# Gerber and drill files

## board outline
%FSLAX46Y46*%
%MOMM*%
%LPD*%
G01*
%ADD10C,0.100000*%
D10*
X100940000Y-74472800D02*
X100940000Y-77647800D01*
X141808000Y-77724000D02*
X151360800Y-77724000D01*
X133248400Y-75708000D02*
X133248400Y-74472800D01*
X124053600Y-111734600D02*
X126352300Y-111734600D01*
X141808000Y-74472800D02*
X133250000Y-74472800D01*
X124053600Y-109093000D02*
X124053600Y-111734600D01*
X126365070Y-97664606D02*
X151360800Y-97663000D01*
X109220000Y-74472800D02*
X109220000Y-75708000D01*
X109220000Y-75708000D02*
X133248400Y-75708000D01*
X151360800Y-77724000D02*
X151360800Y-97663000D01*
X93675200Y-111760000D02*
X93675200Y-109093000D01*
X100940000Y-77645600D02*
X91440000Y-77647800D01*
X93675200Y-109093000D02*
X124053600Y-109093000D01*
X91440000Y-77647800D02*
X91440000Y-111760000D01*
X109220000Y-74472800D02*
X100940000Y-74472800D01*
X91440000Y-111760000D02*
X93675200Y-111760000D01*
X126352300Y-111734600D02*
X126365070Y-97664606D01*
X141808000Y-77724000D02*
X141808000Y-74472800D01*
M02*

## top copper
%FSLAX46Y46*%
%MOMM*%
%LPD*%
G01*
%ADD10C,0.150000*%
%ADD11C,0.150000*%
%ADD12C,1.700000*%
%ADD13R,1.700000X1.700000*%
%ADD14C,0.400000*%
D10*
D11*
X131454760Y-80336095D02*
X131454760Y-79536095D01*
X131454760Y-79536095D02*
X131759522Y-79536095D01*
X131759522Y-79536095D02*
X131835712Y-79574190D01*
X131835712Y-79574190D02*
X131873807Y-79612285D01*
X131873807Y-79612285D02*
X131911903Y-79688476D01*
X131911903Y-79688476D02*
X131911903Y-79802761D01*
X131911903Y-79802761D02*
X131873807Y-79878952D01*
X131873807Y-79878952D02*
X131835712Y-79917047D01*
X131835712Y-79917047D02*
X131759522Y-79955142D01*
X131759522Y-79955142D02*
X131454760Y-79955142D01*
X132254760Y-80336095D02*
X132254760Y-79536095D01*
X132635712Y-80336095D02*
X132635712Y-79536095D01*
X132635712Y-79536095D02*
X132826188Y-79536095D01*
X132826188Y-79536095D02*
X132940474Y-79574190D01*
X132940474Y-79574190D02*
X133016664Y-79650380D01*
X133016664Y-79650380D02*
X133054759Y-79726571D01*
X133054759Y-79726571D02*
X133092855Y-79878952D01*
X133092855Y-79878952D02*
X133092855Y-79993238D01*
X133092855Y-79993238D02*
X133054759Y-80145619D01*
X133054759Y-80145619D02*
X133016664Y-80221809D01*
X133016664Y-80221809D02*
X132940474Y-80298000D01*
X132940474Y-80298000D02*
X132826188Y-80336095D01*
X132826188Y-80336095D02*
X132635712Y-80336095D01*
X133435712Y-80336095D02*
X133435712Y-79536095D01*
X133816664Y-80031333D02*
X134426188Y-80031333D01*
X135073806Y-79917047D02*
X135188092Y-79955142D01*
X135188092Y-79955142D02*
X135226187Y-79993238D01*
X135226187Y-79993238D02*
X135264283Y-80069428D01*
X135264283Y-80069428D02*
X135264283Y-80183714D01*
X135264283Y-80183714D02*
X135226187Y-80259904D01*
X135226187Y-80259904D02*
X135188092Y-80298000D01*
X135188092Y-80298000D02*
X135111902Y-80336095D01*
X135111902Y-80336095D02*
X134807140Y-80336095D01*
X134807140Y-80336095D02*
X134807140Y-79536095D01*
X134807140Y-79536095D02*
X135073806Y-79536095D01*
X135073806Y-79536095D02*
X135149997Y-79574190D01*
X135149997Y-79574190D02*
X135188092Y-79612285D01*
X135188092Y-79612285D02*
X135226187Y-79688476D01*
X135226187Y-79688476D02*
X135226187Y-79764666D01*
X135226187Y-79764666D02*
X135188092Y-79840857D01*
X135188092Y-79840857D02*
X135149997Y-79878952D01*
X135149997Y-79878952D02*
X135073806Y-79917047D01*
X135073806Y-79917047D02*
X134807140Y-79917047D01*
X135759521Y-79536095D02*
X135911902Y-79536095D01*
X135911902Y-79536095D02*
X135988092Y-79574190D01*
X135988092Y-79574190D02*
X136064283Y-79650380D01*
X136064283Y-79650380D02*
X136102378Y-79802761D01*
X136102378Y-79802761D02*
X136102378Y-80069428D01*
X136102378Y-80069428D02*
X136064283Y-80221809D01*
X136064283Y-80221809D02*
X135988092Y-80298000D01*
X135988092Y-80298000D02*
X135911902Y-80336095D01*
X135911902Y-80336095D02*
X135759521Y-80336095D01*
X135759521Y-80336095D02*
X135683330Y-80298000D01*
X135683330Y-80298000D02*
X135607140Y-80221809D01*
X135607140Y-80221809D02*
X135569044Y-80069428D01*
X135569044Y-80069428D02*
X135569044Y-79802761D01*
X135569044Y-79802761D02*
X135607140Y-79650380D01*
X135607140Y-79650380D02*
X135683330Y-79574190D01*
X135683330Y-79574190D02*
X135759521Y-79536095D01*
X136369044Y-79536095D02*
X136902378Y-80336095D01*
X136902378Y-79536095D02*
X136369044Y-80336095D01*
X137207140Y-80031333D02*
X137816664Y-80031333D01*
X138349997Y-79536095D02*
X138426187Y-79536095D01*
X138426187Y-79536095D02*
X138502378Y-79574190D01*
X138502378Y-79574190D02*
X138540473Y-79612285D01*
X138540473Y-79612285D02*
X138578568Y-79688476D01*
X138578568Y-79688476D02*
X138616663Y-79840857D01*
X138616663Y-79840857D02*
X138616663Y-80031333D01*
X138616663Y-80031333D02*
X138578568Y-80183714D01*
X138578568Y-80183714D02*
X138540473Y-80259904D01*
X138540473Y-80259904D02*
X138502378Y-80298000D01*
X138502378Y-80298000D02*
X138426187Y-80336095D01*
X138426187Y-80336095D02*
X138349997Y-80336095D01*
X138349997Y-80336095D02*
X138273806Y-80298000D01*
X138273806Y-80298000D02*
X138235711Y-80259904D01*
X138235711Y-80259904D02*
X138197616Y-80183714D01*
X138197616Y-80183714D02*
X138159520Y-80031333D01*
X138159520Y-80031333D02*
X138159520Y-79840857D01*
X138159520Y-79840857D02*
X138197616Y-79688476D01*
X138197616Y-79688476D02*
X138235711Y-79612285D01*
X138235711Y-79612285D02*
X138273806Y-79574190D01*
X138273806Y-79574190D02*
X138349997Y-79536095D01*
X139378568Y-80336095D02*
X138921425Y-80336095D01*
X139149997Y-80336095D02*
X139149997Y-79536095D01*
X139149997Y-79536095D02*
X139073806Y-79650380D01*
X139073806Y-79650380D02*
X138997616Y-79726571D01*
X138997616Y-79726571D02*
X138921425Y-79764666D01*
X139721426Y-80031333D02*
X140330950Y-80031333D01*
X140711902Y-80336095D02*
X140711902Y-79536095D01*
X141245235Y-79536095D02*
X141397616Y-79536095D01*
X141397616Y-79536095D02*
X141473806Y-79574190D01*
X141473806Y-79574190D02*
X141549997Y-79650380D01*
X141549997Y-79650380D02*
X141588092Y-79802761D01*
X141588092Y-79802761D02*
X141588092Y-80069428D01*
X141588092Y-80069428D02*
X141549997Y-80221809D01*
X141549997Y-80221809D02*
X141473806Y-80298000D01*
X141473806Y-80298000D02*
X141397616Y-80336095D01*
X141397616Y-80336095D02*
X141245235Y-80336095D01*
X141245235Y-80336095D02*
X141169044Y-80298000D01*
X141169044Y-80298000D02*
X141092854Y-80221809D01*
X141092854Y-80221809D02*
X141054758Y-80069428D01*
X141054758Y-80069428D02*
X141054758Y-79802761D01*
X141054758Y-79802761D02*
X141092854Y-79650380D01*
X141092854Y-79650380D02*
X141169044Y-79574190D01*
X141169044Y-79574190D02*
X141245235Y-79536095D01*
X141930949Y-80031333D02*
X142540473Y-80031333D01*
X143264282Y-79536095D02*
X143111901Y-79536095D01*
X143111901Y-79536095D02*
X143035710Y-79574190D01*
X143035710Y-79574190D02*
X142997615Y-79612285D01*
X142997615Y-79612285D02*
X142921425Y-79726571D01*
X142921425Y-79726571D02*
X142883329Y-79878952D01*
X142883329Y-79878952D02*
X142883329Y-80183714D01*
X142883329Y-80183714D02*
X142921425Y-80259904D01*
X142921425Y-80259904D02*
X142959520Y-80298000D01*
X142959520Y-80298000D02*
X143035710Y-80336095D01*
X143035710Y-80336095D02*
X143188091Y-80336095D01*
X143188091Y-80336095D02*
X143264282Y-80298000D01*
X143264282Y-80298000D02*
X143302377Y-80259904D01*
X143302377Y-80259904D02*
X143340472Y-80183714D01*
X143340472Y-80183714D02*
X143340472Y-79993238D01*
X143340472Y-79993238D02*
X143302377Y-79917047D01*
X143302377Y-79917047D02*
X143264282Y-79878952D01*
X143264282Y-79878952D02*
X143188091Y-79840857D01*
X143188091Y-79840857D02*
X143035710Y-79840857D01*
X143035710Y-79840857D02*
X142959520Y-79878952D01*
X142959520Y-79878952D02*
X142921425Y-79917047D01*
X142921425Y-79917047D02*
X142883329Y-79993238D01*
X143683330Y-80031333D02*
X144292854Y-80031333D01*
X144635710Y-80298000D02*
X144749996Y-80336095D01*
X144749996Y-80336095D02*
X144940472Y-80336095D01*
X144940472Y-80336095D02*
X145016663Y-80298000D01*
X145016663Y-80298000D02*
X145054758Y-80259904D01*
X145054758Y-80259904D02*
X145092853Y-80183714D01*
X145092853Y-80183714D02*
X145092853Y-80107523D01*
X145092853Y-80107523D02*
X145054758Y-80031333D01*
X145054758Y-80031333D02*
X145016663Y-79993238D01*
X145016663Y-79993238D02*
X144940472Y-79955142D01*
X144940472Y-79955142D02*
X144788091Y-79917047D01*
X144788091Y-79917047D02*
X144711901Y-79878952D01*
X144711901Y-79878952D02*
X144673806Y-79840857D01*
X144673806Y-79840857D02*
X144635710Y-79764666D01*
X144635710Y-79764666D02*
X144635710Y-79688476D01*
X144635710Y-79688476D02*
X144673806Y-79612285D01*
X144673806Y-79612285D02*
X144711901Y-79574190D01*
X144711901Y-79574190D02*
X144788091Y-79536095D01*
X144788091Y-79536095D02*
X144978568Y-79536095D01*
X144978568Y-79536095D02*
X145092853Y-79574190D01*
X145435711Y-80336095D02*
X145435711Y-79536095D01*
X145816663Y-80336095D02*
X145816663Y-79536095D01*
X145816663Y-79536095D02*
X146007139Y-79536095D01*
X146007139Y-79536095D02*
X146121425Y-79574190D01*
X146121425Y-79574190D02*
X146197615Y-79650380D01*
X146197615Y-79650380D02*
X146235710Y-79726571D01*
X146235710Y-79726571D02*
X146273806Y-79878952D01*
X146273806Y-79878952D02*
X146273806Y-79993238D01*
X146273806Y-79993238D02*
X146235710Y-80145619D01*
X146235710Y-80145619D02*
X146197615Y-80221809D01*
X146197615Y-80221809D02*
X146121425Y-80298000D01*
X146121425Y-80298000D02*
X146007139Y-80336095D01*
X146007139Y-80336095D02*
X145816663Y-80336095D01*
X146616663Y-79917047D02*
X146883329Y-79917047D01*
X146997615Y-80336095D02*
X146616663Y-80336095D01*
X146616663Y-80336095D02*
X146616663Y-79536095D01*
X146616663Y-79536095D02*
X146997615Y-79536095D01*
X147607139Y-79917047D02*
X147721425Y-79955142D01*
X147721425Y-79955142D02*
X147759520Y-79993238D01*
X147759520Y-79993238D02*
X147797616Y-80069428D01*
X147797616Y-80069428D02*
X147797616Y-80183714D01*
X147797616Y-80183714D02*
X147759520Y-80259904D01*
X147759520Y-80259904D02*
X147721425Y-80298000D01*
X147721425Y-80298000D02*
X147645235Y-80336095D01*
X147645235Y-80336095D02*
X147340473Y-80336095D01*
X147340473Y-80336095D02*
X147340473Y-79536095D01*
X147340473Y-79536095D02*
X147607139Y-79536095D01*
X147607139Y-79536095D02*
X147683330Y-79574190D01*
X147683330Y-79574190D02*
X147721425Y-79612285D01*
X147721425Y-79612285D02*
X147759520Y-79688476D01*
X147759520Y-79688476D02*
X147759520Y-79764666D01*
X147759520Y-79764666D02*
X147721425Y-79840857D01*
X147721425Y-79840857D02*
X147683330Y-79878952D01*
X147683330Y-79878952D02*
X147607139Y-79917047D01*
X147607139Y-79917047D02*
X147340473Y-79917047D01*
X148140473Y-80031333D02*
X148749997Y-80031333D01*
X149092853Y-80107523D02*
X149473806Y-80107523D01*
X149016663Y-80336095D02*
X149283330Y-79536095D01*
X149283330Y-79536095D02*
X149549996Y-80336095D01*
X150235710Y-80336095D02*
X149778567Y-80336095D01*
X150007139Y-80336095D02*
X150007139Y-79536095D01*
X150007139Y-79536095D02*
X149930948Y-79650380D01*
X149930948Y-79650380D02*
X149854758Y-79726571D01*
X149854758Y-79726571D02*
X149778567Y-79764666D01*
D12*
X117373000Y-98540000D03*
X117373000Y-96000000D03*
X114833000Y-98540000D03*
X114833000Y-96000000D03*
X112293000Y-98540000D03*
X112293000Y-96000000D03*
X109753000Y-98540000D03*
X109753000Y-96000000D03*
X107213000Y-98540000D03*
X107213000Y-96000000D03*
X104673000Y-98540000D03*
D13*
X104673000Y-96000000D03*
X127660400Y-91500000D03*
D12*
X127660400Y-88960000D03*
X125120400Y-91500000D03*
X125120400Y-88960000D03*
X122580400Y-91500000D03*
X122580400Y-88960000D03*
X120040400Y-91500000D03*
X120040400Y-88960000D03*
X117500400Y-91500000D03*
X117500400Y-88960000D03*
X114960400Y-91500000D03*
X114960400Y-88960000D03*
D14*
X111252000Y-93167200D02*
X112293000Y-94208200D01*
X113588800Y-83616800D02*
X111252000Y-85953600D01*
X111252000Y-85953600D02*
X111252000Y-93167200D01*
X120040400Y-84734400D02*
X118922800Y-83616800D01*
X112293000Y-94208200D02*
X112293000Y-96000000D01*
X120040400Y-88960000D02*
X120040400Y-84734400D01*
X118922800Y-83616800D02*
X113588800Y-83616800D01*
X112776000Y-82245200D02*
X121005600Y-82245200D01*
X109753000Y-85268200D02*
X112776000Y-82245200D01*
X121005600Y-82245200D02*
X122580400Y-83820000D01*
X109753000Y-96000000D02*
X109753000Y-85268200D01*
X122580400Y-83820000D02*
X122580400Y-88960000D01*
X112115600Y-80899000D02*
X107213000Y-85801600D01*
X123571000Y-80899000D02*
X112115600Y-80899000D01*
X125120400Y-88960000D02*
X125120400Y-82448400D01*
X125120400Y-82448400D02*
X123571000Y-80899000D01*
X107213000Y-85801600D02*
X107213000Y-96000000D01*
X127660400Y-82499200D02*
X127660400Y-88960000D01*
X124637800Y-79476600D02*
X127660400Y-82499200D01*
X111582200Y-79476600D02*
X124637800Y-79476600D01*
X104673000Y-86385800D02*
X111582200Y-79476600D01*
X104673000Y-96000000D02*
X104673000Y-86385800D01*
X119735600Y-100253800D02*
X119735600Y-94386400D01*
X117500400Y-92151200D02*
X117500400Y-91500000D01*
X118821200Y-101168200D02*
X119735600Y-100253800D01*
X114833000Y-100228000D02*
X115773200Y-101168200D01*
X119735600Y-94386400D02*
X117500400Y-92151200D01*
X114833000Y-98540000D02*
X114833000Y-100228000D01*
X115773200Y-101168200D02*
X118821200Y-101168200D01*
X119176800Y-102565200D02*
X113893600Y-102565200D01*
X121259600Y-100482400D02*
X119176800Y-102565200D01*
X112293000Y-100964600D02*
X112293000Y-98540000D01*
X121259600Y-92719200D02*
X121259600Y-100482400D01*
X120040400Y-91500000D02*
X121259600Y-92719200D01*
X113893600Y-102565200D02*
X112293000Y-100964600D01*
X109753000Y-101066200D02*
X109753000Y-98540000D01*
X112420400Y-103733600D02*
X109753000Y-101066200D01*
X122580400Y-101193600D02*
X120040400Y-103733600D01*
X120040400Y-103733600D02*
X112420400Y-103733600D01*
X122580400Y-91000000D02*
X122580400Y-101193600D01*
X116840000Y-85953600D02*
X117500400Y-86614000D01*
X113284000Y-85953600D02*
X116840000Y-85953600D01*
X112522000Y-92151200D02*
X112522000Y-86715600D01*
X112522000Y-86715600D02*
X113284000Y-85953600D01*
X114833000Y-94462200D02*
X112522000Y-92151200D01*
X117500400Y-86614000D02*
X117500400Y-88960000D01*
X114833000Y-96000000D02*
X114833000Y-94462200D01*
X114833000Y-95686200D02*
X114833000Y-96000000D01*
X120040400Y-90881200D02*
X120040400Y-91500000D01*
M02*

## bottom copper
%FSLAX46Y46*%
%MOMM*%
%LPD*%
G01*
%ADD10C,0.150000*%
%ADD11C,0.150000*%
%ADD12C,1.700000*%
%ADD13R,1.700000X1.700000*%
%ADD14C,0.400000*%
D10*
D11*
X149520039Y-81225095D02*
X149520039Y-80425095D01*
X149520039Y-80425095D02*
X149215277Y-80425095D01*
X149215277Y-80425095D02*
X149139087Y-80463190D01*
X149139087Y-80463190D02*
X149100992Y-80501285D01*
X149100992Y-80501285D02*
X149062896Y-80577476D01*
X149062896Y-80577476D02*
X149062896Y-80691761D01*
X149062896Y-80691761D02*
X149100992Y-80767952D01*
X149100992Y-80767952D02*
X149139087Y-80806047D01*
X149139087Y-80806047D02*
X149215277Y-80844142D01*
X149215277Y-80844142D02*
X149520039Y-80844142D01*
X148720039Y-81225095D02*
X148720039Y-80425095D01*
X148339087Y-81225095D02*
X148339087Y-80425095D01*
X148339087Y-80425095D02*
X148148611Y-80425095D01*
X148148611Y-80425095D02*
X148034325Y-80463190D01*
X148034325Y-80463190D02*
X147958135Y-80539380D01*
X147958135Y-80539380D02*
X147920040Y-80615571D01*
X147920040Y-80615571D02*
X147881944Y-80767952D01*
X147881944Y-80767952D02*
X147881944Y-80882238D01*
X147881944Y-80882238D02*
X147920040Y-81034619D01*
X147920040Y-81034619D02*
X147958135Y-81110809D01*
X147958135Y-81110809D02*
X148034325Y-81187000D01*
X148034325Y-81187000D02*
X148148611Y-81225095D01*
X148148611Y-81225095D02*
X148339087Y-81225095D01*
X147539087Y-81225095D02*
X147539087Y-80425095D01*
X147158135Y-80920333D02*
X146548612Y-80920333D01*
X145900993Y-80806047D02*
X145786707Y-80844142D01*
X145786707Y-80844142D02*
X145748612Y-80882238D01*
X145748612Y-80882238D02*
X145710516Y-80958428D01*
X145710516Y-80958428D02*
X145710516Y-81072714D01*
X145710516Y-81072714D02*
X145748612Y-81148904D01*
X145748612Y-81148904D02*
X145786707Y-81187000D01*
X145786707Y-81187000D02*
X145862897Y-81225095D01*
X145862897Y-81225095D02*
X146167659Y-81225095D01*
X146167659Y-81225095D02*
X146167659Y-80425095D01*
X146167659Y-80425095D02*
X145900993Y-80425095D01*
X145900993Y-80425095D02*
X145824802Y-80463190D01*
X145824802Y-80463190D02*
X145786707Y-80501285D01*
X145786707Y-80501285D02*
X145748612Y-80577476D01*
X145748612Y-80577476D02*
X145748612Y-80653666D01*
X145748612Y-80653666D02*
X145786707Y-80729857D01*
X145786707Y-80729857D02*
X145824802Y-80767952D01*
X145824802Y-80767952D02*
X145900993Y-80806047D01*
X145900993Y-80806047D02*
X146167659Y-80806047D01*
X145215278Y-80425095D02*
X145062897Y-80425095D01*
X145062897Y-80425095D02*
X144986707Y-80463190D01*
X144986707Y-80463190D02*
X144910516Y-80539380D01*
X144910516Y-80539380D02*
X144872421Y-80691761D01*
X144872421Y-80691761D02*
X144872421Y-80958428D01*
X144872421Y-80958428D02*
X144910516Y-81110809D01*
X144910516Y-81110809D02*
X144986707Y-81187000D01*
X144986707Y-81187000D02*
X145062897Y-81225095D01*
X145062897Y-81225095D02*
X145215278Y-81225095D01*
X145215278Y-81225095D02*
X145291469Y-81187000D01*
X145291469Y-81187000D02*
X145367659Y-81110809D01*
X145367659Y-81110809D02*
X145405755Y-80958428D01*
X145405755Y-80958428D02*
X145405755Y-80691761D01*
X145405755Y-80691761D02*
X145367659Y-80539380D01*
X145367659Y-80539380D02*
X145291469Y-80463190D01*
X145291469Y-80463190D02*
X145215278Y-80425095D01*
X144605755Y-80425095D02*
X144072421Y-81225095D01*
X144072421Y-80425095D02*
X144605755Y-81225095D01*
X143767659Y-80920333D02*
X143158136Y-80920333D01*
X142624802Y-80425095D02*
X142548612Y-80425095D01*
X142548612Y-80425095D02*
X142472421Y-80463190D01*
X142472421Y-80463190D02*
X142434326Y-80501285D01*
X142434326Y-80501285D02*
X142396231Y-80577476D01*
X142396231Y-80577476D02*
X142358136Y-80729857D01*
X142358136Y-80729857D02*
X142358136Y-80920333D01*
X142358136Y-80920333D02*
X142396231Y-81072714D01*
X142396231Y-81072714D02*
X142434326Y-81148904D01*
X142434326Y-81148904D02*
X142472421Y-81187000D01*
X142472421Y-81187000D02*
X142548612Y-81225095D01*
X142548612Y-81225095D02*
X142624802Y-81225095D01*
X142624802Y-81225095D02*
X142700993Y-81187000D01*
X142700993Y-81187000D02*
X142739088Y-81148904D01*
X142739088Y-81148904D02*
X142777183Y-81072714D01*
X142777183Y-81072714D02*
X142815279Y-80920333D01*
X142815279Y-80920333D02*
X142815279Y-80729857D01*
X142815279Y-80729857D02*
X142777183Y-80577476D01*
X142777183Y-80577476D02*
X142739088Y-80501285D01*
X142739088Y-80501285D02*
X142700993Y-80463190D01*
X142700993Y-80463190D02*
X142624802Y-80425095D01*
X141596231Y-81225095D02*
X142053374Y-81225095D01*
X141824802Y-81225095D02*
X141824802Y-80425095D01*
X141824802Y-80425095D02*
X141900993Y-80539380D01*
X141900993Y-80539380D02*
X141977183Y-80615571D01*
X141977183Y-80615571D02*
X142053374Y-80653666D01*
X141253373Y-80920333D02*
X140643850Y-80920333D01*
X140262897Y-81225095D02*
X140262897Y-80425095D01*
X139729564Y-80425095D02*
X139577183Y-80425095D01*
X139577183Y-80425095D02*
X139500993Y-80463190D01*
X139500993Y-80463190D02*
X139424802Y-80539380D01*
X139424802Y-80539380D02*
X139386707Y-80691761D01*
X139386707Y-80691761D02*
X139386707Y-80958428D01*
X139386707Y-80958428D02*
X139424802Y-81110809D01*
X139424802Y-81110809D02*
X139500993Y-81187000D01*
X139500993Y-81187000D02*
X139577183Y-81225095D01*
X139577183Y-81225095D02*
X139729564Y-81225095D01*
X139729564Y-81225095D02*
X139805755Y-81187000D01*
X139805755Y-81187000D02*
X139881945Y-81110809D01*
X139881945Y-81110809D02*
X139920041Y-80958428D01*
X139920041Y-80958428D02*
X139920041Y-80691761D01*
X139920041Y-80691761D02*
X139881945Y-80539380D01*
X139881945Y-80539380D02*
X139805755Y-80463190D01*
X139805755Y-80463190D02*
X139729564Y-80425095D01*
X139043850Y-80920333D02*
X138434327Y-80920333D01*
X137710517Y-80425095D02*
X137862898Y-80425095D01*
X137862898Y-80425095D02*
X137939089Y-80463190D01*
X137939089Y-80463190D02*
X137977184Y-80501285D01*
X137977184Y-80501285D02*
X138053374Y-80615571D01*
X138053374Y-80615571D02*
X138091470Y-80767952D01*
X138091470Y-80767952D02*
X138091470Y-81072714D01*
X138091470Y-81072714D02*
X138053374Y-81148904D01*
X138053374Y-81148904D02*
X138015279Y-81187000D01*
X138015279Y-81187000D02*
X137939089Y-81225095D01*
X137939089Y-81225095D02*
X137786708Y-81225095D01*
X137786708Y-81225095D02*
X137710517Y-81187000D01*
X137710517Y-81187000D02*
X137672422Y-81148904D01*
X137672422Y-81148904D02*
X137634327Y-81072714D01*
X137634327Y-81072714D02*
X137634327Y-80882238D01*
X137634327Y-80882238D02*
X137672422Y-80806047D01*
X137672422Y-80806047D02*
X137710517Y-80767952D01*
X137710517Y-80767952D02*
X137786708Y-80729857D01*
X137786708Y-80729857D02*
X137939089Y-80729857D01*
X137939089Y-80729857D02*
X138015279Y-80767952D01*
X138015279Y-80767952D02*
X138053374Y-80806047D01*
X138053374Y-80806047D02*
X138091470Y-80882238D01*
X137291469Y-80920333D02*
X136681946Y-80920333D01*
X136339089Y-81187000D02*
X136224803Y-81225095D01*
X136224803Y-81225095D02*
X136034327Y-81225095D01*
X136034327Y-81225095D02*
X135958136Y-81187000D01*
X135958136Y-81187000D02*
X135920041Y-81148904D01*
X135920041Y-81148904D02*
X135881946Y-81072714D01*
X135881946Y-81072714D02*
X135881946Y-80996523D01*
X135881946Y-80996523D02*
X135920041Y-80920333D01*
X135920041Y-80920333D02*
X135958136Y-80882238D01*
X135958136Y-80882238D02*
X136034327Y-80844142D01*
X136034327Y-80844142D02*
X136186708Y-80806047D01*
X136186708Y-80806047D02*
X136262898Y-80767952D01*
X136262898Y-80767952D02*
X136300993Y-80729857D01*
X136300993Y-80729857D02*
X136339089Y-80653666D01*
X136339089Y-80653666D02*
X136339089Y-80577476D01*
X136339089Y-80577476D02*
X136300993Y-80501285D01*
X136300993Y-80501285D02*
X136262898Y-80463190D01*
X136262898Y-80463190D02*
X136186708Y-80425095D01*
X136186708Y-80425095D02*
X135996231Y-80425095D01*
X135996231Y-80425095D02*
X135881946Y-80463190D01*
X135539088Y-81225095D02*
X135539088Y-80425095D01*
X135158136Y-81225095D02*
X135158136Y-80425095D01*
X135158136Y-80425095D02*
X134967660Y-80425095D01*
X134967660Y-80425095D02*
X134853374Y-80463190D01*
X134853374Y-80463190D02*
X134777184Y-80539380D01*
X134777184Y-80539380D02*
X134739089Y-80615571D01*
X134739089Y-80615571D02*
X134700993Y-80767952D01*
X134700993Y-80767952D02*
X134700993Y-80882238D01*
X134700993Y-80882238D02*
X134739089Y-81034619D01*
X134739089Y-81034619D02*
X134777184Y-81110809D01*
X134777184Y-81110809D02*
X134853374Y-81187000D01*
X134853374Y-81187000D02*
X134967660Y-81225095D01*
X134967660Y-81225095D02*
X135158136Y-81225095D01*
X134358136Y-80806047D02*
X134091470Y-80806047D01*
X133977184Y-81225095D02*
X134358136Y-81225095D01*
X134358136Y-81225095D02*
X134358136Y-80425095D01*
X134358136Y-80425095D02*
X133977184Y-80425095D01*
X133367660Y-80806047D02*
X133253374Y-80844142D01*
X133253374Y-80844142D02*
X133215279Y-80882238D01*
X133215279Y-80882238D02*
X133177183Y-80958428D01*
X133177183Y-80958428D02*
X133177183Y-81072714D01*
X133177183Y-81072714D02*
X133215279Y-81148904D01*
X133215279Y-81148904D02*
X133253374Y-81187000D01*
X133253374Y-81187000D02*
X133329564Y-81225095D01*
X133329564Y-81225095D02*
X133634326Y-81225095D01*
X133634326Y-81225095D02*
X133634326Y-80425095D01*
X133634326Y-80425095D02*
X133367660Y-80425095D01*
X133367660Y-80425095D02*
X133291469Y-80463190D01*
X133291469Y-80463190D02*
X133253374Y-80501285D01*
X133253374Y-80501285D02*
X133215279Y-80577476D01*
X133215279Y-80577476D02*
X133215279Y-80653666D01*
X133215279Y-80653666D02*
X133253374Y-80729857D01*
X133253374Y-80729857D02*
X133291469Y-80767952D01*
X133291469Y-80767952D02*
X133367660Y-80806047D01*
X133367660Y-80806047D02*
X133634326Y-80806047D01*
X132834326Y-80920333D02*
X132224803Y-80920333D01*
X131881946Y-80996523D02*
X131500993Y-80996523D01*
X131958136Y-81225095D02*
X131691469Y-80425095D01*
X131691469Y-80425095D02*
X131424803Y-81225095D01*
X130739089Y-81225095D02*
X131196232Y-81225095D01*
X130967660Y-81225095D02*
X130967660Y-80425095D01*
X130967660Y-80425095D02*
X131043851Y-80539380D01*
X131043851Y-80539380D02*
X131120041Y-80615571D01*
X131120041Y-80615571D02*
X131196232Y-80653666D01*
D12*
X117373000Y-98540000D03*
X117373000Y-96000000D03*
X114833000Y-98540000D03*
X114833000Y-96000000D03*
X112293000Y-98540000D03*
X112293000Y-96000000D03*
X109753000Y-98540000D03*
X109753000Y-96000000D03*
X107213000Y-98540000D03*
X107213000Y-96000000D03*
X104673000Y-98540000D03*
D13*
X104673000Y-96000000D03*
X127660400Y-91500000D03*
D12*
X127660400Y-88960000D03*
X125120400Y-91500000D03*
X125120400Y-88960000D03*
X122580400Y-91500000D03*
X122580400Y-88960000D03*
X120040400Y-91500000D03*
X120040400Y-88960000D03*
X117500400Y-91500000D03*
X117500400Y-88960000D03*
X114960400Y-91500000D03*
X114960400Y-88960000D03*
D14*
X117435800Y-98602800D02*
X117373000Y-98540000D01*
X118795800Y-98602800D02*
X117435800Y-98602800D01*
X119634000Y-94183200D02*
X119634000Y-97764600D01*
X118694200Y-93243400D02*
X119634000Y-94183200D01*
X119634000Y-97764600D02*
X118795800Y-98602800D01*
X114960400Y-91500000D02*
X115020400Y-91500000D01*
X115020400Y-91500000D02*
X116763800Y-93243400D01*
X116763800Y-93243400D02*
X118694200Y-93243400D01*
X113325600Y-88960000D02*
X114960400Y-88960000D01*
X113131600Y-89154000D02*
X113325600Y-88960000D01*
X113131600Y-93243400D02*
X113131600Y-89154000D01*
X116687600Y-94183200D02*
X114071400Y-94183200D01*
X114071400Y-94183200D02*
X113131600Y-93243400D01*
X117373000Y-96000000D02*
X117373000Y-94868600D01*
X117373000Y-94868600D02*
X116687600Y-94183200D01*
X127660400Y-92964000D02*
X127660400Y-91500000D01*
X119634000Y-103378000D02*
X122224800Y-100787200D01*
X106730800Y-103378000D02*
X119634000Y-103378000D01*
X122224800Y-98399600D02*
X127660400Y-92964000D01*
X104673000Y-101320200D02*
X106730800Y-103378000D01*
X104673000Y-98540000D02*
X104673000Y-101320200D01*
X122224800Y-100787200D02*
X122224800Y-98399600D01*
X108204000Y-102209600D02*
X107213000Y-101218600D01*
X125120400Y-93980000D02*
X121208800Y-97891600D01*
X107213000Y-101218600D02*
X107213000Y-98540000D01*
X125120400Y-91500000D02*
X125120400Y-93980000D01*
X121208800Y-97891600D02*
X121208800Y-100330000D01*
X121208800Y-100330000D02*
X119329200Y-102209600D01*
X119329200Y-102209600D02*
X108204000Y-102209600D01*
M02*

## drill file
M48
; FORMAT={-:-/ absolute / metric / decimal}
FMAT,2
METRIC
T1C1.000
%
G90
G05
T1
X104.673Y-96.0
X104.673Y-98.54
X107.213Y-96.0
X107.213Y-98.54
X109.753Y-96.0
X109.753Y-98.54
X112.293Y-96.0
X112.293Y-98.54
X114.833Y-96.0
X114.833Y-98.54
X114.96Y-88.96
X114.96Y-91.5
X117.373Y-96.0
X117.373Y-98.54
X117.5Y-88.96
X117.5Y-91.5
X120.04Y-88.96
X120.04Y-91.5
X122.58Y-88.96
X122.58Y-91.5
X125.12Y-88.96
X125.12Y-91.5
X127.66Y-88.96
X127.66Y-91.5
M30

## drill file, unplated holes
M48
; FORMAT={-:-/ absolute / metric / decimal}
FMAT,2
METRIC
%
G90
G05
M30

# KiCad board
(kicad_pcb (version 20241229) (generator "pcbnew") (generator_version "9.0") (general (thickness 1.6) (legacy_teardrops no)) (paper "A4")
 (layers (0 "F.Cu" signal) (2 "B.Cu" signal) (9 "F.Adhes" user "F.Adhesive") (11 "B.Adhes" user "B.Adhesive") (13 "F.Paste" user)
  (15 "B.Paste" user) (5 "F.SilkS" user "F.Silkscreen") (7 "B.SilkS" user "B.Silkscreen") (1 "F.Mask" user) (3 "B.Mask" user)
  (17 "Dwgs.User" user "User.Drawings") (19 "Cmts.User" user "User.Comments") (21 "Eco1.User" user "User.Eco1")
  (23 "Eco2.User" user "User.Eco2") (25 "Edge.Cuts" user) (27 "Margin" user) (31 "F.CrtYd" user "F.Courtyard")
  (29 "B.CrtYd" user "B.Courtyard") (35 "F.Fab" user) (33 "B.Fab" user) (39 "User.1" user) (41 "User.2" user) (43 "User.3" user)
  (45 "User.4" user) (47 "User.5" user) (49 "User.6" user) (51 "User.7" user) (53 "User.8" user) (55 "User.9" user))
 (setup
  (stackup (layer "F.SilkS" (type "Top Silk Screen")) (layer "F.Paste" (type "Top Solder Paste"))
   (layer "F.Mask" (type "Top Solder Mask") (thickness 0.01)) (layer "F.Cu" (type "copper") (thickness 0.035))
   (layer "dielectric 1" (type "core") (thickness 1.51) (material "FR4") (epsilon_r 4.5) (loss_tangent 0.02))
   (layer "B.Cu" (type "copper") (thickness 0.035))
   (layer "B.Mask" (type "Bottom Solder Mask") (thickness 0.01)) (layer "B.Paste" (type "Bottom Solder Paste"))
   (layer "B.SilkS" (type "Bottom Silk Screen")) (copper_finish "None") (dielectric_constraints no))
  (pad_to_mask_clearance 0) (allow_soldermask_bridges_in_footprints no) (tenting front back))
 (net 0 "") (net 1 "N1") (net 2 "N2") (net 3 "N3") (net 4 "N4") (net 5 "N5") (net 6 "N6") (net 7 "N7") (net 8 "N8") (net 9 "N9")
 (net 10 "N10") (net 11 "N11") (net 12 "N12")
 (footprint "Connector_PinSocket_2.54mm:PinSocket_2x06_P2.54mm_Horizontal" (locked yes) (layer "F.Cu") (at 127.6604 91.5 -90)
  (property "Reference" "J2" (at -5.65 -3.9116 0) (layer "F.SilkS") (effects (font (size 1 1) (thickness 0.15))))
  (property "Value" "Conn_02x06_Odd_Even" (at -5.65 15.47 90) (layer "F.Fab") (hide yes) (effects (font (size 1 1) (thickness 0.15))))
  (pad "1" thru_hole rect (at 0 0 270) (size 1.7 1.7) (drill 1) (layers "*.Cu" "*.Mask") (remove_unused_layers no) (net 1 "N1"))
  (pad "2" thru_hole circle (at -2.54 0 270) (size 1.7 1.7) (drill 1) (layers "*.Cu" "*.Mask") (remove_unused_layers no) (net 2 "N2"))
  (pad "3" thru_hole circle (at 0 2.54 270) (size 1.7 1.7) (drill 1) (layers "*.Cu" "*.Mask") (remove_unused_layers no) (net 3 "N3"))
  (pad "4" thru_hole circle (at -2.54 2.54 270) (size 1.7 1.7) (drill 1) (layers "*.Cu" "*.Mask") (remove_unused_layers no) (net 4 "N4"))
  (pad "5" thru_hole circle (at 0 5.08 270) (size 1.7 1.7) (drill 1) (layers "*.Cu" "*.Mask") (remove_unused_layers no) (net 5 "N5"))
  (pad "6" thru_hole circle (at -2.54 5.08 270) (size 1.7 1.7) (drill 1) (layers "*.Cu" "*.Mask") (remove_unused_layers no) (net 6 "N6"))
  (pad "7" thru_hole circle (at 0 7.62 270) (size 1.7 1.7) (drill 1) (layers "*.Cu" "*.Mask") (remove_unused_layers no) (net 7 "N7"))
  (pad "8" thru_hole circle (at -2.54 7.62 270) (size 1.7 1.7) (drill 1) (layers "*.Cu" "*.Mask") (remove_unused_layers no) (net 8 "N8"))
  (pad "9" thru_hole circle (at 0 10.16 270) (size 1.7 1.7) (drill 1) (layers "*.Cu" "*.Mask") (remove_unused_layers no) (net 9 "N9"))
  (pad "10" thru_hole circle (at -2.54 10.16 270) (size 1.7 1.7) (drill 1) (layers "*.Cu" "*.Mask") (remove_unused_layers no) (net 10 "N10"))
  (pad "11" thru_hole circle (at 0 12.7 270) (size 1.7 1.7) (drill 1) (layers "*.Cu" "*.Mask") (remove_unused_layers no) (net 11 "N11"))
  (pad "12" thru_hole circle (at -2.54 12.7 270) (size 1.7 1.7) (drill 1) (layers "*.Cu" "*.Mask") (remove_unused_layers no) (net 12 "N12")))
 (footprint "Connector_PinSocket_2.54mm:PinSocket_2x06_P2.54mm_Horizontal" (layer "F.Cu") (at 104.673 96 90)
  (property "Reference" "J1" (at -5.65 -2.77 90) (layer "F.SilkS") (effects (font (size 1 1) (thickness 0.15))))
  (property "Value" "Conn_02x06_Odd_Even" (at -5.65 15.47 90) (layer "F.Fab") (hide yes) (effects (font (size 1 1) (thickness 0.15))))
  (pad "1" thru_hole rect (at 0 0 90) (size 1.7 1.7) (drill 1) (layers "*.Cu" "*.Mask") (remove_unused_layers no) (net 2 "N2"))
  (pad "2" thru_hole circle (at -2.54 0 90) (size 1.7 1.7) (drill 1) (layers "*.Cu" "*.Mask") (remove_unused_layers no) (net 1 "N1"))
  (pad "3" thru_hole circle (at 0 2.54 90) (size 1.7 1.7) (drill 1) (layers "*.Cu" "*.Mask") (remove_unused_layers no) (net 4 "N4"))
  (pad "4" thru_hole circle (at -2.54 2.54 90) (size 1.7 1.7) (drill 1) (layers "*.Cu" "*.Mask") (remove_unused_layers no) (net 3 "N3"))
  (pad "5" thru_hole circle (at 0 5.08 90) (size 1.7 1.7) (drill 1) (layers "*.Cu" "*.Mask") (remove_unused_layers no) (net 6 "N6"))
  (pad "6" thru_hole circle (at -2.54 5.08 90) (size 1.7 1.7) (drill 1) (layers "*.Cu" "*.Mask") (remove_unused_layers no) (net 5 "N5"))
  (pad "7" thru_hole circle (at 0 7.62 90) (size 1.7 1.7) (drill 1) (layers "*.Cu" "*.Mask") (remove_unused_layers no) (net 8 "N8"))
  (pad "8" thru_hole circle (at -2.54 7.62 90) (size 1.7 1.7) (drill 1) (layers "*.Cu" "*.Mask") (remove_unused_layers no) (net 7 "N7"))
  (pad "9" thru_hole circle (at 0 10.16 90) (size 1.7 1.7) (drill 1) (layers "*.Cu" "*.Mask") (remove_unused_layers no) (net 10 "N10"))
  (pad "10" thru_hole circle (at -2.54 10.16 90) (size 1.7 1.7) (drill 1) (layers "*.Cu" "*.Mask") (remove_unused_layers no) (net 9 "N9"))
  (pad "11" thru_hole circle (at 0 12.7 90) (size 1.7 1.7) (drill 1) (layers "*.Cu" "*.Mask") (remove_unused_layers no) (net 12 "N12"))
  (pad "12" thru_hole circle (at -2.54 12.7 90) (size 1.7 1.7) (drill 1) (layers "*.Cu" "*.Mask") (remove_unused_layers no) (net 11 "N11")))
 (gr_line (start 100.9396 74.4728) (end 100.9396 77.6732) (stroke (width 0.1) (type default)) (locked yes) (layer "Edge.Cuts"))
 (gr_line (start 141.808 77.724) (end 151.3608 77.724) (stroke (width 0.1) (type default)) (locked yes) (layer "Edge.Cuts"))
 (gr_line (start 133.2484 75.708) (end 133.25 74.4728) (stroke (width 0.1) (type default)) (locked yes) (layer "Edge.Cuts"))
 (gr_line (start 124.0536 111.76) (end 126.352277 111.76) (stroke (width 0.1) (type default)) (locked yes) (layer "Edge.Cuts"))
 (gr_line (start 141.808 74.4728) (end 133.2484 74.4728) (stroke (width 0.1) (type solid)) (locked yes) (layer "Edge.Cuts"))
 (gr_line (start 124.0536 109.093) (end 124.0536 111.76) (stroke (width 0.1) (type default)) (locked yes) (layer "Edge.Cuts"))
 (gr_line (start 126.36507 97.664606) (end 151.3608 97.663) (stroke (width 0.1) (type default)) (locked yes) (layer "Edge.Cuts"))
 (gr_line (start 109.22 74.4728) (end 109.22 75.708) (stroke (width 0.1) (type default)) (locked yes) (layer "Edge.Cuts"))
 (gr_line (start 109.22 75.708) (end 133.2484 75.708) (stroke (width 0.1) (type default)) (locked yes) (layer "Edge.Cuts"))
 (gr_line (start 151.3608 77.724) (end 151.3608 97.663) (stroke (width 0.1) (type default)) (locked yes) (layer "Edge.Cuts"))
 (gr_line (start 93.6752 111.76) (end 93.6752 109.093) (stroke (width 0.1) (type default)) (locked yes) (layer "Edge.Cuts"))
 (gr_line (start 100.9396 77.6732) (end 91.44 77.6732) (stroke (width 0.1) (type default)) (locked yes) (layer "Edge.Cuts"))
 (gr_line (start 93.6752 109.093) (end 124.0536 109.093) (stroke (width 0.1) (type default)) (locked yes) (layer "Edge.Cuts"))
 (gr_line (start 91.44 77.6732) (end 91.44 111.76) (stroke (width 0.1) (type default)) (locked yes) (layer "Edge.Cuts"))
 (gr_line (start 109.22 74.4728) (end 100.9396 74.4728) (stroke (width 0.1) (type default)) (locked yes) (layer "Edge.Cuts"))
 (gr_line (start 91.44 111.76) (end 93.6752 111.76) (stroke (width 0.1) (type default)) (locked yes) (layer "Edge.Cuts"))
 (gr_line (start 126.3523 111.76) (end 126.36507 97.664606) (stroke (width 0.1) (type default)) (locked yes) (layer "Edge.Cuts"))
 (gr_line (start 141.808 77.724) (end 141.808 74.4728) (stroke (width 0.1) (type default)) (locked yes) (layer "Edge.Cuts"))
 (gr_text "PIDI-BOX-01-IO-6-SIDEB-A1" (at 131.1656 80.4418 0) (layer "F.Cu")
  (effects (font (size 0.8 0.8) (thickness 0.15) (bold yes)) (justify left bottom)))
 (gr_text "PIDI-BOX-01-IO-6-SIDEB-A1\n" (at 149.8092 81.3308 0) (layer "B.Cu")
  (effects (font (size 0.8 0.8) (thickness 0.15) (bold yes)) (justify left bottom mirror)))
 (segment (start 119.1768 102.5652) (end 113.8936 102.5652) (width 0.4) (layer "F.Cu") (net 7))
 (segment (start 121.2596 100.4824) (end 119.1768 102.5652) (width 0.4) (layer "F.Cu") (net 7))
 (segment (start 120.0404 90.8812) (end 120.0404 91.5) (width 0.4) (layer "F.Cu") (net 7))
 (segment (start 113.8936 102.5652) (end 112.293 100.9646) (width 0.4) (layer "F.Cu") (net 7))
 (segment (start 120.0404 91.5) (end 121.2596 92.7192) (width 0.4) (layer "F.Cu") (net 7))
 (segment (start 121.2596 92.7192) (end 121.2596 100.4824) (width 0.4) (layer "F.Cu") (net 7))
 (segment (start 112.293 100.9646) (end 112.293 98.54) (width 0.4) (layer "F.Cu") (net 7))
 (segment (start 124.6378 79.4766) (end 127.6604 82.4992) (width 0.4) (layer "F.Cu") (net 2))
 (segment (start 104.673 86.3858) (end 111.5822 79.4766) (width 0.4) (layer "F.Cu") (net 2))
 (segment (start 104.673 96) (end 104.673 86.3858) (width 0.4) (layer "F.Cu") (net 2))
 (segment (start 127.6604 82.4992) (end 127.6604 88.96) (width 0.4) (layer "F.Cu") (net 2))
 (segment (start 111.5822 79.4766) (end 124.6378 79.4766) (width 0.4) (layer "F.Cu") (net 2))
 (segment (start 109.753 85.2682) (end 112.776 82.2452) (width 0.4) (layer "F.Cu") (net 6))
 (segment (start 109.753 96) (end 109.753 85.2682) (width 0.4) (layer "F.Cu") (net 6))
 (segment (start 121.0056 82.2452) (end 122.5804 83.82) (width 0.4) (layer "F.Cu") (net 6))
 (segment (start 112.776 82.2452) (end 121.0056 82.2452) (width 0.4) (layer "F.Cu") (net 6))
 (segment (start 122.5804 83.82) (end 122.5804 88.96) (width 0.4) (layer "F.Cu") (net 6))
 (segment (start 121.2088 97.8916) (end 121.2088 100.33) (width 0.4) (layer "B.Cu") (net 3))
 (segment (start 119.3292 102.2096) (end 108.204 102.2096) (width 0.4) (layer "B.Cu") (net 3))
 (segment (start 125.1204 91.5) (end 125.1204 93.98) (width 0.4) (layer "B.Cu") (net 3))
 (segment (start 108.204 102.2096) (end 107.213 101.2186) (width 0.4) (layer "B.Cu") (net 3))
 (segment (start 125.1204 93.98) (end 121.2088 97.8916) (width 0.4) (layer "B.Cu") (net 3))
 (segment (start 107.213 101.2186) (end 107.213 98.54) (width 0.4) (layer "B.Cu") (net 3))
 (segment (start 121.2088 100.33) (end 119.3292 102.2096) (width 0.4) (layer "B.Cu") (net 3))
 (segment (start 116.84 85.9536) (end 117.5004 86.614) (width 0.4) (layer "F.Cu") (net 10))
 (segment (start 114.833 96) (end 114.833 94.4622) (width 0.4) (layer "F.Cu") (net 10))
 (segment (start 114.833 95.6862) (end 114.833 96) (width 0.4) (layer "F.Cu") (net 10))
 (segment (start 113.284 85.9536) (end 116.84 85.9536) (width 0.4) (layer "F.Cu") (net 10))
 (segment (start 114.833 94.4622) (end 112.522 92.1512) (width 0.4) (layer "F.Cu") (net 10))
 (segment (start 112.522 86.7156) (end 113.284 85.9536) (width 0.4) (layer "F.Cu") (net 10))
 (segment (start 112.522 92.1512) (end 112.522 86.7156) (width 0.4) (layer "F.Cu") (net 10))
 (segment (start 117.5004 86.614) (end 117.5004 88.96) (width 0.4) (layer "F.Cu") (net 10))
 (segment (start 119.7356 100.2538) (end 119.7356 94.3864) (width 0.4) (layer "F.Cu") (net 9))
 (segment (start 114.833 98.54) (end 114.833 100.228) (width 0.4) (layer "F.Cu") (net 9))
 (segment (start 118.8212 101.1682) (end 119.7356 100.2538) (width 0.4) (layer "F.Cu") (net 9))
 (segment (start 115.7732 101.1682) (end 118.8212 101.1682) (width 0.4) (layer "F.Cu") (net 9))
 (segment (start 114.833 100.228) (end 115.7732 101.1682) (width 0.4) (layer "F.Cu") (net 9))
 (segment (start 119.7356 94.3864) (end 117.5004 92.1512) (width 0.4) (layer "F.Cu") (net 9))
 (segment (start 117.5004 92.1512) (end 117.5004 91.5) (width 0.4) (layer "F.Cu") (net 9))
 (segment (start 113.1316 89.154) (end 113.3256 88.96) (width 0.4) (layer "B.Cu") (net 12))
 (segment (start 113.1316 93.2434) (end 113.1316 89.154) (width 0.4) (layer "B.Cu") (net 12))
 (segment (start 117.373 96) (end 117.373 94.8686) (width 0.4) (layer "B.Cu") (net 12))
 (segment (start 116.6876 94.1832) (end 114.0714 94.1832) (width 0.4) (layer "B.Cu") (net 12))
 (segment (start 113.3256 88.96) (end 114.9604 88.96) (width 0.4) (layer "B.Cu") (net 12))
 (segment (start 117.373 94.8686) (end 116.6876 94.1832) (width 0.4) (layer "B.Cu") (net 12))
 (segment (start 114.0714 94.1832) (end 113.1316 93.2434) (width 0.4) (layer "B.Cu") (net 12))
 (segment (start 125.1204 82.4484) (end 123.571 80.899) (width 0.4) (layer "F.Cu") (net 4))
 (segment (start 123.571 80.899) (end 112.1156 80.899) (width 0.4) (layer "F.Cu") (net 4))
 (segment (start 125.1204 88.96) (end 125.1204 82.4484) (width 0.4) (layer "F.Cu") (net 4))
 (segment (start 112.1156 80.899) (end 107.213 85.8016) (width 0.4) (layer "F.Cu") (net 4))
 (segment (start 107.213 85.8016) (end 107.213 96) (width 0.4) (layer "F.Cu") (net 4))
 (segment (start 112.4204 103.7336) (end 109.753 101.0662) (width 0.4) (layer "F.Cu") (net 5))
 (segment (start 122.5804 91) (end 122.5804 101.1936) (width 0.4) (layer "F.Cu") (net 5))
 (segment (start 120.0404 103.7336) (end 112.4204 103.7336) (width 0.4) (layer "F.Cu") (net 5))
 (segment (start 109.753 101.0662) (end 109.753 98.54) (width 0.4) (layer "F.Cu") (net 5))
 (segment (start 122.5804 101.1936) (end 120.0404 103.7336) (width 0.4) (layer "F.Cu") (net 5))
 (segment (start 104.673 98.54) (end 104.673 101.3202) (width 0.4) (layer "B.Cu") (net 1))
 (segment (start 119.634 103.378) (end 122.2248 100.7872) (width 0.4) (layer "B.Cu") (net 1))
 (segment (start 104.673 101.3202) (end 106.7308 103.378) (width 0.4) (layer "B.Cu") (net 1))
 (segment (start 122.2248 98.3996) (end 127.6604 92.964) (width 0.4) (layer "B.Cu") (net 1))
 (segment (start 122.2248 100.7872) (end 122.2248 98.3996) (width 0.4) (layer "B.Cu") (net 1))
 (segment (start 127.6604 92.964) (end 127.6604 91.5) (width 0.4) (layer "B.Cu") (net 1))
 (segment (start 106.7308 103.378) (end 119.634 103.378) (width 0.4) (layer "B.Cu") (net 1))
 (segment (start 118.6942 93.2434) (end 119.634 94.1832) (width 0.4) (layer "B.Cu") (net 11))
 (segment (start 119.634 94.1832) (end 119.634 97.7646) (width 0.4) (layer "B.Cu") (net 11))
 (segment (start 118.7958 98.6028) (end 117.4358 98.6028) (width 0.4) (layer "B.Cu") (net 11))
 (segment (start 116.7638 93.2434) (end 118.6942 93.2434) (width 0.4) (layer "B.Cu") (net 11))
 (segment (start 114.9604 91.5) (end 115.0204 91.5) (width 0.4) (layer "B.Cu") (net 11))
 (segment (start 117.4358 98.6028) (end 117.373 98.54) (width 0.4) (layer "B.Cu") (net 11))
 (segment (start 115.0204 91.5) (end 116.7638 93.2434) (width 0.4) (layer "B.Cu") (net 11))
 (segment (start 119.634 97.7646) (end 118.7958 98.6028) (width 0.4) (layer "B.Cu") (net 11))
 (segment (start 111.252 93.1672) (end 112.293 94.2082) (width 0.4) (layer "F.Cu") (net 8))
 (segment (start 120.0404 84.7344) (end 118.9228 83.6168) (width 0.4) (layer "F.Cu") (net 8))
 (segment (start 112.293 94.2082) (end 112.293 96) (width 0.4) (layer "F.Cu") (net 8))
 (segment (start 118.9228 83.6168) (end 113.5888 83.6168) (width 0.4) (layer "F.Cu") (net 8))
 (segment (start 111.252 85.9536) (end 111.252 93.1672) (width 0.4) (layer "F.Cu") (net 8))
 (segment (start 120.0404 88.96) (end 120.0404 84.7344) (width 0.4) (layer "F.Cu") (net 8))
 (segment (start 113.5888 83.6168) (end 111.252 85.9536) (width 0.4) (layer "F.Cu") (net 8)))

